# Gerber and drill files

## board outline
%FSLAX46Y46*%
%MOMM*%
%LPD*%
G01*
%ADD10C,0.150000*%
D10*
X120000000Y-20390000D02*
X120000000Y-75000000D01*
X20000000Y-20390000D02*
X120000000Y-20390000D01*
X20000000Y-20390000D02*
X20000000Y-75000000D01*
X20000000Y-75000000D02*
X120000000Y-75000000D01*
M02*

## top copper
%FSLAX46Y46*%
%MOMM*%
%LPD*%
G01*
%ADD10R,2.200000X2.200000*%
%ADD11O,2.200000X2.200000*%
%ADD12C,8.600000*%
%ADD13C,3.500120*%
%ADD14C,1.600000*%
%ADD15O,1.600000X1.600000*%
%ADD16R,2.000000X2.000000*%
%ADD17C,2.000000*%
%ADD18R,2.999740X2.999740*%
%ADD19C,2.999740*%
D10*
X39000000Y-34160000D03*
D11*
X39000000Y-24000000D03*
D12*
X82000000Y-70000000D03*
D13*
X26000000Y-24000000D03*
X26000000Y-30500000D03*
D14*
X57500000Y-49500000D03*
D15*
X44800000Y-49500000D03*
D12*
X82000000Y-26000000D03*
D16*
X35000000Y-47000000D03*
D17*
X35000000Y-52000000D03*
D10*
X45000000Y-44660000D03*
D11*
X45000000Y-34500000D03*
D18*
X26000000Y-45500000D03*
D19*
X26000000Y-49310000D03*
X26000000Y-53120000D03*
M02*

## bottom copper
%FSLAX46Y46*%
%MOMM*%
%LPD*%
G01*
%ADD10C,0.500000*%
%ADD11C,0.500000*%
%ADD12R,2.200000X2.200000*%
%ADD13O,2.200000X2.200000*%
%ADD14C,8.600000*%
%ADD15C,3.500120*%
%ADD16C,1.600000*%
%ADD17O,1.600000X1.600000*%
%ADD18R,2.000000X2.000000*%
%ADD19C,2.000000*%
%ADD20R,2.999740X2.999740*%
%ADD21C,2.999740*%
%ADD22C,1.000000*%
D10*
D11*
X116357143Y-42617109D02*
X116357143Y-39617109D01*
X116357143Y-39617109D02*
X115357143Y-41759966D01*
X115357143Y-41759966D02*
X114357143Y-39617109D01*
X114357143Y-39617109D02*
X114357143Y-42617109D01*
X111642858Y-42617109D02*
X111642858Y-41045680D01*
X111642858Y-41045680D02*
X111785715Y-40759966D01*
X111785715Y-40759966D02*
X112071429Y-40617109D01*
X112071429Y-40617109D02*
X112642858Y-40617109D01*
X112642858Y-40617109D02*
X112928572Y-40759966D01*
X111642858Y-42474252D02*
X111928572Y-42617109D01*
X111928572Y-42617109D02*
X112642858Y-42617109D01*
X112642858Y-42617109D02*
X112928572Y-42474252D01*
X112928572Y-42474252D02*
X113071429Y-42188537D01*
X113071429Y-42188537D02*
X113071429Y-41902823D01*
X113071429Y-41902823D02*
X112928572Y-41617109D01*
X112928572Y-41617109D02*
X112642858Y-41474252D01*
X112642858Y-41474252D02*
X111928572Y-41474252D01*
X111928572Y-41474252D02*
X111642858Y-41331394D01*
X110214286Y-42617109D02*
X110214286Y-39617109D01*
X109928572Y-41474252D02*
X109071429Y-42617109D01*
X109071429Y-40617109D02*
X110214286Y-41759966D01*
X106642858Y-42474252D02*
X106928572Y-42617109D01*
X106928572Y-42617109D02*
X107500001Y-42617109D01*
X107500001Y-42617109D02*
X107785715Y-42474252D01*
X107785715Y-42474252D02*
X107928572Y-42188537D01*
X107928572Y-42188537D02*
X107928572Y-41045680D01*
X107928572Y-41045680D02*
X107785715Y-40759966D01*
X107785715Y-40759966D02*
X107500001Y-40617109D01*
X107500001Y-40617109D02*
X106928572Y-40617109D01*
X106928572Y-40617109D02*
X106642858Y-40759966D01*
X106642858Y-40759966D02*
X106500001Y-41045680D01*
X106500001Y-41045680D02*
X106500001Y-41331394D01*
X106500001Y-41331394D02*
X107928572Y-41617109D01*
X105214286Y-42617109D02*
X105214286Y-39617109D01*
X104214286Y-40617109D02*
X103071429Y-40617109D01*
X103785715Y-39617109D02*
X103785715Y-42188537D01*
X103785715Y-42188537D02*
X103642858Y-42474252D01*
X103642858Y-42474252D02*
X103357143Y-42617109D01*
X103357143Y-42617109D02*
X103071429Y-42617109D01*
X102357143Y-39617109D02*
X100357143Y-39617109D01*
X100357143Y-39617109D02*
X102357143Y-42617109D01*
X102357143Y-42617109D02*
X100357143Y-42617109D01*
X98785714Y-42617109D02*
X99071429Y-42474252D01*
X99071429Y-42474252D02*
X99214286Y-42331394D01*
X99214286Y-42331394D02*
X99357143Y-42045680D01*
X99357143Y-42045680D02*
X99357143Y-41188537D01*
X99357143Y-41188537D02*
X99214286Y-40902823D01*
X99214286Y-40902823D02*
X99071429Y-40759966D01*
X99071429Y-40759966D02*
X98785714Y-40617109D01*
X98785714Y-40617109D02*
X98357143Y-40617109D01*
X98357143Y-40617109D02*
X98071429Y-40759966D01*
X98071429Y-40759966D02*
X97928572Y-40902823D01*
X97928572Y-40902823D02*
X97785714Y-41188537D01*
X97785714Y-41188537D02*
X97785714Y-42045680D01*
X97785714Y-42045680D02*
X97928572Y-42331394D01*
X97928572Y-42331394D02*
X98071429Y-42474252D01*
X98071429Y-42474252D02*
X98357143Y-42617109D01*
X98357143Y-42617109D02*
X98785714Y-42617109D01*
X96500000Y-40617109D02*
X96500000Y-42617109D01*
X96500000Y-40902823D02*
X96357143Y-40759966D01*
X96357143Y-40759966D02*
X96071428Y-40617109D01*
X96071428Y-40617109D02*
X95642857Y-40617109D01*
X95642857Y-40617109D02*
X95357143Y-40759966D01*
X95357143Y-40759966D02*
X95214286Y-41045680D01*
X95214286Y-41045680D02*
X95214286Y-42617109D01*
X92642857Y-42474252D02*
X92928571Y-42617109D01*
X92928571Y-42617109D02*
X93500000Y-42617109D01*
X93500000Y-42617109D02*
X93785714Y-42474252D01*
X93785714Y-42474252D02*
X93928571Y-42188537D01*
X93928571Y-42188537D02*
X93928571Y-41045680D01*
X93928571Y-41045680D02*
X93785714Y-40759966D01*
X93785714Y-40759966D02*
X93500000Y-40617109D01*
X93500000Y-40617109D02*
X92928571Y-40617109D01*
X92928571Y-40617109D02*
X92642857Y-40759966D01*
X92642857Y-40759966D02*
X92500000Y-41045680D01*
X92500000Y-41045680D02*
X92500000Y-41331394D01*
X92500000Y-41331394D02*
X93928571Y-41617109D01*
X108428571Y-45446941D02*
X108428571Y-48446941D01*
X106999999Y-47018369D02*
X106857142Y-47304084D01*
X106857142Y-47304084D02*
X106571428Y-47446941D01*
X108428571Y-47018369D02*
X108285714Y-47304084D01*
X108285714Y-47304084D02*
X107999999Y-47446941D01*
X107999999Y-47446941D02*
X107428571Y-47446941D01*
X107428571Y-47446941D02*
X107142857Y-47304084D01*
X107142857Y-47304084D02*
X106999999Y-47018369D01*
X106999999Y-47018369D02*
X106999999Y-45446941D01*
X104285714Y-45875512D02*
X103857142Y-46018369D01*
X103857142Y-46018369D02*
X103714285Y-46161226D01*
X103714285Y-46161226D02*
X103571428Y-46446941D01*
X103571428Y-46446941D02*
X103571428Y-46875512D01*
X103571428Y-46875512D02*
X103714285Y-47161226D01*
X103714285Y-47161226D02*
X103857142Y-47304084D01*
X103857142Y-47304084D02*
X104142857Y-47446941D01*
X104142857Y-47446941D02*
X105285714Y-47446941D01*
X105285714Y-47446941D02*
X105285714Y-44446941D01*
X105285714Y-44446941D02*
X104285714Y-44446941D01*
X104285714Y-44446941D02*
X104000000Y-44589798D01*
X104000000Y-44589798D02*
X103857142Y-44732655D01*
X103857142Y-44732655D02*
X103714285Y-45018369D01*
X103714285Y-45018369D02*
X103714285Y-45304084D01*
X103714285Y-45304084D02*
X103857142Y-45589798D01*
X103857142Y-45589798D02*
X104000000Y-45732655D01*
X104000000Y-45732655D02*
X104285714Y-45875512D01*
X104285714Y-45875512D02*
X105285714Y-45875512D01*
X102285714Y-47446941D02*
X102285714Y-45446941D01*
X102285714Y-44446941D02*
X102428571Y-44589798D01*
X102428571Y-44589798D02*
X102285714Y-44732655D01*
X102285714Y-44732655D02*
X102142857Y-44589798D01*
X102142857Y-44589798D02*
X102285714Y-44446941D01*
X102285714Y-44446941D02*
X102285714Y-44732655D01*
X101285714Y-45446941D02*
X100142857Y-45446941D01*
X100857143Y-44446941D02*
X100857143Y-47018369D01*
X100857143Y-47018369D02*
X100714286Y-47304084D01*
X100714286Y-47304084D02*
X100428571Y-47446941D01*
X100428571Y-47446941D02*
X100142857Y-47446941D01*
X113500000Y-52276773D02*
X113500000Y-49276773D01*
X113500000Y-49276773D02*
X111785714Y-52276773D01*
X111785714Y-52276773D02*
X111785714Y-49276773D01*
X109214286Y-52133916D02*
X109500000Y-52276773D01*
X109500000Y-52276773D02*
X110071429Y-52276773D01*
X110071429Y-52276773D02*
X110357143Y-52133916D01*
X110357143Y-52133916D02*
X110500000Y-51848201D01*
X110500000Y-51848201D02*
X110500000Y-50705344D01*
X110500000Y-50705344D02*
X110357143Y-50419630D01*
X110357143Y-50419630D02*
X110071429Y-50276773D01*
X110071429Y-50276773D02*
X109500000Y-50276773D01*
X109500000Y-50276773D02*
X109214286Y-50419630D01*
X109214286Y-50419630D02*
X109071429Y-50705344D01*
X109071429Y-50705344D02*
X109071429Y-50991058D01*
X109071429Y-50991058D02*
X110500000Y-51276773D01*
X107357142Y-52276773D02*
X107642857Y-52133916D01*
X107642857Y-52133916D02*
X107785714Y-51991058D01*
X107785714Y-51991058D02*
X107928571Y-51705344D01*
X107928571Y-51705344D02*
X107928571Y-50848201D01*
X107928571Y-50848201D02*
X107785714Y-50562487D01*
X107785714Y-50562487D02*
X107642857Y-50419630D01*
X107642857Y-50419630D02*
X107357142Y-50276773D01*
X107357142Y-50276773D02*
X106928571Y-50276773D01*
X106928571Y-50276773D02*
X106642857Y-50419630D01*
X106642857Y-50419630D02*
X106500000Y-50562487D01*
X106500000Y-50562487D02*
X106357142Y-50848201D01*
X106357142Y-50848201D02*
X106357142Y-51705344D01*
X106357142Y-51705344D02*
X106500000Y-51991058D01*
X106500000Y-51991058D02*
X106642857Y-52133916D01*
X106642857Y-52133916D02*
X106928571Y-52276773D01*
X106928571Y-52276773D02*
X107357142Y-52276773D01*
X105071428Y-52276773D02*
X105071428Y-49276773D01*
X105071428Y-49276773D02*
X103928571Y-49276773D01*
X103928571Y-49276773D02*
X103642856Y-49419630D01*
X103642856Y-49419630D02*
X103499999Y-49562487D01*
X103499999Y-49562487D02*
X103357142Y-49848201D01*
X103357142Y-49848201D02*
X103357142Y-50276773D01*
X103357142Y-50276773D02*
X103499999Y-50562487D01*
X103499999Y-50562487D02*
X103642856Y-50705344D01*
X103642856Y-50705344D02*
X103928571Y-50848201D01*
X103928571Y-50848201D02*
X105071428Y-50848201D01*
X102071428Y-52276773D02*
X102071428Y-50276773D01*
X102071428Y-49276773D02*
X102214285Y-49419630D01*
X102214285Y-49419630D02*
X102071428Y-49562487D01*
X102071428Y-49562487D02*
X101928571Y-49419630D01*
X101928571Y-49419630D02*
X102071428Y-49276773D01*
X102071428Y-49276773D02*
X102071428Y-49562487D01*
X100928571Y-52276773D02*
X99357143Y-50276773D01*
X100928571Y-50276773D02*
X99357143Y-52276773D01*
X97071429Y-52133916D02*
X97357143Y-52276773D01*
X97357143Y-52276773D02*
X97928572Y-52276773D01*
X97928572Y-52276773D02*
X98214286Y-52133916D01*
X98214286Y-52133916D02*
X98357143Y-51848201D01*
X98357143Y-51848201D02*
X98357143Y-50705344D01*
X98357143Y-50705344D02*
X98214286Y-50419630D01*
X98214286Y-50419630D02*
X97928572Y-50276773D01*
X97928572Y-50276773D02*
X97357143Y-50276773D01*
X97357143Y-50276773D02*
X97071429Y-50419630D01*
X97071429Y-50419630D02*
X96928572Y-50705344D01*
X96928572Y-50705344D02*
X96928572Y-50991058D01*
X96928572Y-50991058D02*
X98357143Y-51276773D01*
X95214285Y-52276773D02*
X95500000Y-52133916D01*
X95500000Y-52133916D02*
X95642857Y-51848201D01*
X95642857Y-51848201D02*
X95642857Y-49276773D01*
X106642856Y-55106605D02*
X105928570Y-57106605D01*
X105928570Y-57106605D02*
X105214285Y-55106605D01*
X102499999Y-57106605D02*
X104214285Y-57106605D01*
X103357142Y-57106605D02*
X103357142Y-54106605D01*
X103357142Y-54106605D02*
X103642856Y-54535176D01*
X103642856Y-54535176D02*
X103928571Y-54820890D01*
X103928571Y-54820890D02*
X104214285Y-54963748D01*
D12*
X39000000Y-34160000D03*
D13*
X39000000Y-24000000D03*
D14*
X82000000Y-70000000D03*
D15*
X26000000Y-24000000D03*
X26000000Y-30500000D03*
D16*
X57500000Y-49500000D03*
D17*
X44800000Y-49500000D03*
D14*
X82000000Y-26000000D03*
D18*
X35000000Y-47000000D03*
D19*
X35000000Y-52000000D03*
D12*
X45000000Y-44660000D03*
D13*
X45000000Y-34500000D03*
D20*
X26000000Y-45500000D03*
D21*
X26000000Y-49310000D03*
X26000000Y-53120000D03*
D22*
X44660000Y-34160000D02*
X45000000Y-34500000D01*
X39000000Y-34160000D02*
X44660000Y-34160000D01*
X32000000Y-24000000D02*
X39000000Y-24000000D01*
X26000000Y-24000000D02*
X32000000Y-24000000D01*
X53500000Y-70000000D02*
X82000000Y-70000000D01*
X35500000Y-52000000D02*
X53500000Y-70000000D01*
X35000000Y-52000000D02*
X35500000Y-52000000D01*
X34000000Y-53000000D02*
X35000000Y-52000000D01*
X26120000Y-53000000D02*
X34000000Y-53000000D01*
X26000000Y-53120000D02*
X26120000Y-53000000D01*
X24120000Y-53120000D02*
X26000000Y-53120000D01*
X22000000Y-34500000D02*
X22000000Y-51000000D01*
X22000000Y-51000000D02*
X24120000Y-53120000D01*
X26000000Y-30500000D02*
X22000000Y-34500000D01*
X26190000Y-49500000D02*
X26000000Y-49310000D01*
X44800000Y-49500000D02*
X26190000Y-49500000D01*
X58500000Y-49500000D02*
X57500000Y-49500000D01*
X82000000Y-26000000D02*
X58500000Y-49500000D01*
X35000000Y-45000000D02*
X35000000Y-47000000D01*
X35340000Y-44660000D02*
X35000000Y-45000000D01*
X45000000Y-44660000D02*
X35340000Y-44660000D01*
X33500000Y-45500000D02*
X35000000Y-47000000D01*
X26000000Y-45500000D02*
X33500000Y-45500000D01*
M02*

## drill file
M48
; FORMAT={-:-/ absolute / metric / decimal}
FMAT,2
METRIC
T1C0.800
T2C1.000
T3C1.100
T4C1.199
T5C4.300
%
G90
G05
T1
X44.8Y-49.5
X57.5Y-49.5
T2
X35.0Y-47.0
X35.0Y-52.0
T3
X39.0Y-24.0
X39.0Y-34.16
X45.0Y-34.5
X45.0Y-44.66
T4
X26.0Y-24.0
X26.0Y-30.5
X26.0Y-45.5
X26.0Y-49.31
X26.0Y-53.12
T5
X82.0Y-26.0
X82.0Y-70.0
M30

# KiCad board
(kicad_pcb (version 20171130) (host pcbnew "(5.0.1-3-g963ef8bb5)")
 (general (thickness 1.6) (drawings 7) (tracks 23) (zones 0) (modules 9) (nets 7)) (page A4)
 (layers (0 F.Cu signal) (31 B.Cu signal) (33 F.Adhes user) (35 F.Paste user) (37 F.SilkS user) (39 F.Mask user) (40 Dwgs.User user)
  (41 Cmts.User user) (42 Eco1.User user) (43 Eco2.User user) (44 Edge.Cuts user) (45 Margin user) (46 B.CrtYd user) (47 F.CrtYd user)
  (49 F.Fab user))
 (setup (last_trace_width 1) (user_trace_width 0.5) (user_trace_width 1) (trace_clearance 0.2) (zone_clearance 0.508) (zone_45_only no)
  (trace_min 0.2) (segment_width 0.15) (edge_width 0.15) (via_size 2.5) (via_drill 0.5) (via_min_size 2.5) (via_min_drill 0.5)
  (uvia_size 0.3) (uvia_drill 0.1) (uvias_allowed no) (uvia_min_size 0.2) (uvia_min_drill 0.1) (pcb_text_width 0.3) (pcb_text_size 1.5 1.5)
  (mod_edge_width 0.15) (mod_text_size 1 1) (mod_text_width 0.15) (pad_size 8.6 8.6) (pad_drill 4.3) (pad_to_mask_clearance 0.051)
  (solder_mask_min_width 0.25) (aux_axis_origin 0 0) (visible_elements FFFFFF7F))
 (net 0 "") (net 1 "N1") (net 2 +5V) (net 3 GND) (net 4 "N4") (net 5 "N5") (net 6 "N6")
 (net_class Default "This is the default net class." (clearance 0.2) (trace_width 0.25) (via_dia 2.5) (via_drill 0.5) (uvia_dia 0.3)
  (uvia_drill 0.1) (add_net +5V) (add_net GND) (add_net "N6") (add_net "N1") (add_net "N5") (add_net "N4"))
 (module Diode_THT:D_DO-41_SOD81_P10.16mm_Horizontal (layer F.Cu) (at 39 34.16 90)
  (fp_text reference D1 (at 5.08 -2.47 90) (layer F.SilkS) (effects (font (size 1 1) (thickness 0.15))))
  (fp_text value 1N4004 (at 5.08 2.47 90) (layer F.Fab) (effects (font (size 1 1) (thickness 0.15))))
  (pad 1 thru_hole rect (at 0 0 90) (size 2.2 2.2) (drill 1.1) (layers *.Cu *.Mask) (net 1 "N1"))
  (pad 2 thru_hole oval (at 10.16 0 90) (size 2.2 2.2) (drill 1.1) (layers *.Cu *.Mask) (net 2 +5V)))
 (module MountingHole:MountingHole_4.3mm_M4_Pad (layer F.Cu) (at 82 70)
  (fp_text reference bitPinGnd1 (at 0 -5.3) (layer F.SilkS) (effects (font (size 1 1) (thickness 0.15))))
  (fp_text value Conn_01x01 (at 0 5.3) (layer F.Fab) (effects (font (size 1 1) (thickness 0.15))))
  (pad 1 thru_hole circle (at 0 0) (size 8.6 8.6) (drill 4.3) (layers *.Cu *.Mask) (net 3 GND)))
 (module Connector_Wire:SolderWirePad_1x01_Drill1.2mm (layer F.Cu) (at 26 24 270)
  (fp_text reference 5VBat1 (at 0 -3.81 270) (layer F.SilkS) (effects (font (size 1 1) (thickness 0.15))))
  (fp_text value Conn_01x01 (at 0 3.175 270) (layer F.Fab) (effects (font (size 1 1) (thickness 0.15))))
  (pad 1 thru_hole circle (at 0 0 270) (size 3.50012 3.50012) (drill 1.19888) (layers *.Cu *.Mask) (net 2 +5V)))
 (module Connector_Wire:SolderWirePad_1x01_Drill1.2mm (layer F.Cu) (at 26 30.5 270)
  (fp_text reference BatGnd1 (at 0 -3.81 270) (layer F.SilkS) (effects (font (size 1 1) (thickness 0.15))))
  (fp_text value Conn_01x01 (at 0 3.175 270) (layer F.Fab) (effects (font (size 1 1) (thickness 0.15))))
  (pad 1 thru_hole circle (at 0 0 270) (size 3.50012 3.50012) (drill 1.19888) (layers *.Cu *.Mask) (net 3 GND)))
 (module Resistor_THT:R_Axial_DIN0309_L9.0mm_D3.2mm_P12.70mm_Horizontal (layer F.Cu) (at 57.5 49.5 180)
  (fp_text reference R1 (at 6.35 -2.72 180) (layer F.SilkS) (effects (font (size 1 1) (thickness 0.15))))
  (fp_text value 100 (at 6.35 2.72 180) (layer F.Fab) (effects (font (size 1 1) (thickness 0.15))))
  (pad 1 thru_hole circle (at 0 0 180) (size 1.6 1.6) (drill 0.8) (layers *.Cu *.Mask) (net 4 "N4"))
  (pad 2 thru_hole oval (at 12.7 0 180) (size 1.6 1.6) (drill 0.8) (layers *.Cu *.Mask) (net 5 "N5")))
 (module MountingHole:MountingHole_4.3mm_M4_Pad (layer F.Cu) (at 82 26)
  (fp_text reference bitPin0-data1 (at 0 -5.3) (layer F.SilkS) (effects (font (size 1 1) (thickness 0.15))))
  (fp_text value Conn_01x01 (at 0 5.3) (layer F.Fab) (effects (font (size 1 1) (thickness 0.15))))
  (pad 1 thru_hole circle (at 0 0) (size 8.6 8.6) (drill 4.3) (layers *.Cu *.Mask) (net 4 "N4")))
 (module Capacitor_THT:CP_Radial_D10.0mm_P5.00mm (layer F.Cu) (at 35 47 270)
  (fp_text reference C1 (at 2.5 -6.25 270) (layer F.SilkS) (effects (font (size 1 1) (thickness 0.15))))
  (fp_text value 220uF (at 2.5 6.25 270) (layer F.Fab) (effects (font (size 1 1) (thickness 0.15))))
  (pad 1 thru_hole rect (at 0 0 270) (size 2 2) (drill 1) (layers *.Cu *.Mask) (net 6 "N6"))
  (pad 2 thru_hole circle (at 5 0 270) (size 2 2) (drill 1) (layers *.Cu *.Mask) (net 3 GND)))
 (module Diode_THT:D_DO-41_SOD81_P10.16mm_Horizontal (layer F.Cu) (at 45 44.66 90)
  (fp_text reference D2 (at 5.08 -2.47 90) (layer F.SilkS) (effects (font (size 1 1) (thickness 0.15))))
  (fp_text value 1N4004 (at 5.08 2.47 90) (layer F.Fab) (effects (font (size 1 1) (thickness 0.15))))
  (pad 1 thru_hole rect (at 0 0 90) (size 2.2 2.2) (drill 1.1) (layers *.Cu *.Mask) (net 6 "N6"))
  (pad 2 thru_hole oval (at 10.16 0 90) (size 2.2 2.2) (drill 1.1) (layers *.Cu *.Mask) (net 1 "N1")))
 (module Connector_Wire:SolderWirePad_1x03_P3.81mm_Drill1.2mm (layer F.Cu) (at 26 45.5 270)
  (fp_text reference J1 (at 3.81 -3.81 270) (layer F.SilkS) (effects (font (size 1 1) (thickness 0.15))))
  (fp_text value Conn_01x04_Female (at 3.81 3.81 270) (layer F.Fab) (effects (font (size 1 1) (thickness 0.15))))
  (pad 1 thru_hole rect (at 0 0 270) (size 2.99974 2.99974) (drill 1.19888) (layers *.Cu *.Mask) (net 6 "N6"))
  (pad 2 thru_hole circle (at 3.81 0 270) (size 2.99974 2.99974) (drill 1.19888) (layers *.Cu *.Mask) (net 5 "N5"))
  (pad 3 thru_hole circle (at 7.62 0 270) (size 2.99974 2.99974) (drill 1.19888) (layers *.Cu *.Mask) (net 3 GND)))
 (gr_line (start 120 20.39) (end 120 75) (layer Edge.Cuts) (width 0.15))
 (gr_line (start 20 20.39) (end 120 20.39) (layer Edge.Cuts) (width 0.15))
 (gr_line (start 20 20.39) (end 20 75) (layer Edge.Cuts) (width 0.15))
 (gr_line (start 20 75) (end 120 75) (layer Edge.Cuts) (width 0.15))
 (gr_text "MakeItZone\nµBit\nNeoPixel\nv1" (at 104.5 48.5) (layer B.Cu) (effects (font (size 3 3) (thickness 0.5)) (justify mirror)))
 (segment (start 44.66 34.16) (end 45 34.5) (width 1) (layer B.Cu) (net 1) (status 30))
 (segment (start 39 34.16) (end 44.66 34.16) (width 1) (layer B.Cu) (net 1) (status 30))
 (segment (start 32 24) (end 39 24) (width 1) (layer B.Cu) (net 2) (status 20))
 (segment (start 26 24) (end 32 24) (width 1) (layer B.Cu) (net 2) (status 10))
 (segment (start 53.5 70) (end 82 70) (width 1) (layer B.Cu) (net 3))
 (segment (start 35.5 52) (end 53.5 70) (width 1) (layer B.Cu) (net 3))
 (segment (start 35 52) (end 35.5 52) (width 1) (layer B.Cu) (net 3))
 (segment (start 34 53) (end 35 52) (width 1) (layer B.Cu) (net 3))
 (segment (start 26.12 53) (end 34 53) (width 1) (layer B.Cu) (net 3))
 (segment (start 26 53.12) (end 26.12 53) (width 1) (layer B.Cu) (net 3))
 (segment (start 24.12 53.12) (end 26 53.12) (width 1) (layer B.Cu) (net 3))
 (segment (start 22 34.5) (end 22 51) (width 1) (layer B.Cu) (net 3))
 (segment (start 22 51) (end 24.12 53.12) (width 1) (layer B.Cu) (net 3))
 (segment (start 26 30.5) (end 22 34.5) (width 1) (layer B.Cu) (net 3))
 (segment (start 26.19 49.5) (end 26 49.31) (width 1) (layer B.Cu) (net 5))
 (segment (start 44.8 49.5) (end 26.19 49.5) (width 1) (layer B.Cu) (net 5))
 (segment (start 58.5 49.5) (end 57.5 49.5) (width 1) (layer B.Cu) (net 4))
 (segment (start 82 26) (end 58.5 49.5) (width 1) (layer B.Cu) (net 4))
 (segment (start 35 45) (end 35 47) (width 1) (layer B.Cu) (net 6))
 (segment (start 35.34 44.66) (end 35 45) (width 1) (layer B.Cu) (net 6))
 (segment (start 45 44.66) (end 35.34 44.66) (width 1) (layer B.Cu) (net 6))
 (segment (start 33.5 45.5) (end 35 47) (width 1) (layer B.Cu) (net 6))
 (segment (start 26 45.5) (end 33.5 45.5) (width 1) (layer B.Cu) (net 6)))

